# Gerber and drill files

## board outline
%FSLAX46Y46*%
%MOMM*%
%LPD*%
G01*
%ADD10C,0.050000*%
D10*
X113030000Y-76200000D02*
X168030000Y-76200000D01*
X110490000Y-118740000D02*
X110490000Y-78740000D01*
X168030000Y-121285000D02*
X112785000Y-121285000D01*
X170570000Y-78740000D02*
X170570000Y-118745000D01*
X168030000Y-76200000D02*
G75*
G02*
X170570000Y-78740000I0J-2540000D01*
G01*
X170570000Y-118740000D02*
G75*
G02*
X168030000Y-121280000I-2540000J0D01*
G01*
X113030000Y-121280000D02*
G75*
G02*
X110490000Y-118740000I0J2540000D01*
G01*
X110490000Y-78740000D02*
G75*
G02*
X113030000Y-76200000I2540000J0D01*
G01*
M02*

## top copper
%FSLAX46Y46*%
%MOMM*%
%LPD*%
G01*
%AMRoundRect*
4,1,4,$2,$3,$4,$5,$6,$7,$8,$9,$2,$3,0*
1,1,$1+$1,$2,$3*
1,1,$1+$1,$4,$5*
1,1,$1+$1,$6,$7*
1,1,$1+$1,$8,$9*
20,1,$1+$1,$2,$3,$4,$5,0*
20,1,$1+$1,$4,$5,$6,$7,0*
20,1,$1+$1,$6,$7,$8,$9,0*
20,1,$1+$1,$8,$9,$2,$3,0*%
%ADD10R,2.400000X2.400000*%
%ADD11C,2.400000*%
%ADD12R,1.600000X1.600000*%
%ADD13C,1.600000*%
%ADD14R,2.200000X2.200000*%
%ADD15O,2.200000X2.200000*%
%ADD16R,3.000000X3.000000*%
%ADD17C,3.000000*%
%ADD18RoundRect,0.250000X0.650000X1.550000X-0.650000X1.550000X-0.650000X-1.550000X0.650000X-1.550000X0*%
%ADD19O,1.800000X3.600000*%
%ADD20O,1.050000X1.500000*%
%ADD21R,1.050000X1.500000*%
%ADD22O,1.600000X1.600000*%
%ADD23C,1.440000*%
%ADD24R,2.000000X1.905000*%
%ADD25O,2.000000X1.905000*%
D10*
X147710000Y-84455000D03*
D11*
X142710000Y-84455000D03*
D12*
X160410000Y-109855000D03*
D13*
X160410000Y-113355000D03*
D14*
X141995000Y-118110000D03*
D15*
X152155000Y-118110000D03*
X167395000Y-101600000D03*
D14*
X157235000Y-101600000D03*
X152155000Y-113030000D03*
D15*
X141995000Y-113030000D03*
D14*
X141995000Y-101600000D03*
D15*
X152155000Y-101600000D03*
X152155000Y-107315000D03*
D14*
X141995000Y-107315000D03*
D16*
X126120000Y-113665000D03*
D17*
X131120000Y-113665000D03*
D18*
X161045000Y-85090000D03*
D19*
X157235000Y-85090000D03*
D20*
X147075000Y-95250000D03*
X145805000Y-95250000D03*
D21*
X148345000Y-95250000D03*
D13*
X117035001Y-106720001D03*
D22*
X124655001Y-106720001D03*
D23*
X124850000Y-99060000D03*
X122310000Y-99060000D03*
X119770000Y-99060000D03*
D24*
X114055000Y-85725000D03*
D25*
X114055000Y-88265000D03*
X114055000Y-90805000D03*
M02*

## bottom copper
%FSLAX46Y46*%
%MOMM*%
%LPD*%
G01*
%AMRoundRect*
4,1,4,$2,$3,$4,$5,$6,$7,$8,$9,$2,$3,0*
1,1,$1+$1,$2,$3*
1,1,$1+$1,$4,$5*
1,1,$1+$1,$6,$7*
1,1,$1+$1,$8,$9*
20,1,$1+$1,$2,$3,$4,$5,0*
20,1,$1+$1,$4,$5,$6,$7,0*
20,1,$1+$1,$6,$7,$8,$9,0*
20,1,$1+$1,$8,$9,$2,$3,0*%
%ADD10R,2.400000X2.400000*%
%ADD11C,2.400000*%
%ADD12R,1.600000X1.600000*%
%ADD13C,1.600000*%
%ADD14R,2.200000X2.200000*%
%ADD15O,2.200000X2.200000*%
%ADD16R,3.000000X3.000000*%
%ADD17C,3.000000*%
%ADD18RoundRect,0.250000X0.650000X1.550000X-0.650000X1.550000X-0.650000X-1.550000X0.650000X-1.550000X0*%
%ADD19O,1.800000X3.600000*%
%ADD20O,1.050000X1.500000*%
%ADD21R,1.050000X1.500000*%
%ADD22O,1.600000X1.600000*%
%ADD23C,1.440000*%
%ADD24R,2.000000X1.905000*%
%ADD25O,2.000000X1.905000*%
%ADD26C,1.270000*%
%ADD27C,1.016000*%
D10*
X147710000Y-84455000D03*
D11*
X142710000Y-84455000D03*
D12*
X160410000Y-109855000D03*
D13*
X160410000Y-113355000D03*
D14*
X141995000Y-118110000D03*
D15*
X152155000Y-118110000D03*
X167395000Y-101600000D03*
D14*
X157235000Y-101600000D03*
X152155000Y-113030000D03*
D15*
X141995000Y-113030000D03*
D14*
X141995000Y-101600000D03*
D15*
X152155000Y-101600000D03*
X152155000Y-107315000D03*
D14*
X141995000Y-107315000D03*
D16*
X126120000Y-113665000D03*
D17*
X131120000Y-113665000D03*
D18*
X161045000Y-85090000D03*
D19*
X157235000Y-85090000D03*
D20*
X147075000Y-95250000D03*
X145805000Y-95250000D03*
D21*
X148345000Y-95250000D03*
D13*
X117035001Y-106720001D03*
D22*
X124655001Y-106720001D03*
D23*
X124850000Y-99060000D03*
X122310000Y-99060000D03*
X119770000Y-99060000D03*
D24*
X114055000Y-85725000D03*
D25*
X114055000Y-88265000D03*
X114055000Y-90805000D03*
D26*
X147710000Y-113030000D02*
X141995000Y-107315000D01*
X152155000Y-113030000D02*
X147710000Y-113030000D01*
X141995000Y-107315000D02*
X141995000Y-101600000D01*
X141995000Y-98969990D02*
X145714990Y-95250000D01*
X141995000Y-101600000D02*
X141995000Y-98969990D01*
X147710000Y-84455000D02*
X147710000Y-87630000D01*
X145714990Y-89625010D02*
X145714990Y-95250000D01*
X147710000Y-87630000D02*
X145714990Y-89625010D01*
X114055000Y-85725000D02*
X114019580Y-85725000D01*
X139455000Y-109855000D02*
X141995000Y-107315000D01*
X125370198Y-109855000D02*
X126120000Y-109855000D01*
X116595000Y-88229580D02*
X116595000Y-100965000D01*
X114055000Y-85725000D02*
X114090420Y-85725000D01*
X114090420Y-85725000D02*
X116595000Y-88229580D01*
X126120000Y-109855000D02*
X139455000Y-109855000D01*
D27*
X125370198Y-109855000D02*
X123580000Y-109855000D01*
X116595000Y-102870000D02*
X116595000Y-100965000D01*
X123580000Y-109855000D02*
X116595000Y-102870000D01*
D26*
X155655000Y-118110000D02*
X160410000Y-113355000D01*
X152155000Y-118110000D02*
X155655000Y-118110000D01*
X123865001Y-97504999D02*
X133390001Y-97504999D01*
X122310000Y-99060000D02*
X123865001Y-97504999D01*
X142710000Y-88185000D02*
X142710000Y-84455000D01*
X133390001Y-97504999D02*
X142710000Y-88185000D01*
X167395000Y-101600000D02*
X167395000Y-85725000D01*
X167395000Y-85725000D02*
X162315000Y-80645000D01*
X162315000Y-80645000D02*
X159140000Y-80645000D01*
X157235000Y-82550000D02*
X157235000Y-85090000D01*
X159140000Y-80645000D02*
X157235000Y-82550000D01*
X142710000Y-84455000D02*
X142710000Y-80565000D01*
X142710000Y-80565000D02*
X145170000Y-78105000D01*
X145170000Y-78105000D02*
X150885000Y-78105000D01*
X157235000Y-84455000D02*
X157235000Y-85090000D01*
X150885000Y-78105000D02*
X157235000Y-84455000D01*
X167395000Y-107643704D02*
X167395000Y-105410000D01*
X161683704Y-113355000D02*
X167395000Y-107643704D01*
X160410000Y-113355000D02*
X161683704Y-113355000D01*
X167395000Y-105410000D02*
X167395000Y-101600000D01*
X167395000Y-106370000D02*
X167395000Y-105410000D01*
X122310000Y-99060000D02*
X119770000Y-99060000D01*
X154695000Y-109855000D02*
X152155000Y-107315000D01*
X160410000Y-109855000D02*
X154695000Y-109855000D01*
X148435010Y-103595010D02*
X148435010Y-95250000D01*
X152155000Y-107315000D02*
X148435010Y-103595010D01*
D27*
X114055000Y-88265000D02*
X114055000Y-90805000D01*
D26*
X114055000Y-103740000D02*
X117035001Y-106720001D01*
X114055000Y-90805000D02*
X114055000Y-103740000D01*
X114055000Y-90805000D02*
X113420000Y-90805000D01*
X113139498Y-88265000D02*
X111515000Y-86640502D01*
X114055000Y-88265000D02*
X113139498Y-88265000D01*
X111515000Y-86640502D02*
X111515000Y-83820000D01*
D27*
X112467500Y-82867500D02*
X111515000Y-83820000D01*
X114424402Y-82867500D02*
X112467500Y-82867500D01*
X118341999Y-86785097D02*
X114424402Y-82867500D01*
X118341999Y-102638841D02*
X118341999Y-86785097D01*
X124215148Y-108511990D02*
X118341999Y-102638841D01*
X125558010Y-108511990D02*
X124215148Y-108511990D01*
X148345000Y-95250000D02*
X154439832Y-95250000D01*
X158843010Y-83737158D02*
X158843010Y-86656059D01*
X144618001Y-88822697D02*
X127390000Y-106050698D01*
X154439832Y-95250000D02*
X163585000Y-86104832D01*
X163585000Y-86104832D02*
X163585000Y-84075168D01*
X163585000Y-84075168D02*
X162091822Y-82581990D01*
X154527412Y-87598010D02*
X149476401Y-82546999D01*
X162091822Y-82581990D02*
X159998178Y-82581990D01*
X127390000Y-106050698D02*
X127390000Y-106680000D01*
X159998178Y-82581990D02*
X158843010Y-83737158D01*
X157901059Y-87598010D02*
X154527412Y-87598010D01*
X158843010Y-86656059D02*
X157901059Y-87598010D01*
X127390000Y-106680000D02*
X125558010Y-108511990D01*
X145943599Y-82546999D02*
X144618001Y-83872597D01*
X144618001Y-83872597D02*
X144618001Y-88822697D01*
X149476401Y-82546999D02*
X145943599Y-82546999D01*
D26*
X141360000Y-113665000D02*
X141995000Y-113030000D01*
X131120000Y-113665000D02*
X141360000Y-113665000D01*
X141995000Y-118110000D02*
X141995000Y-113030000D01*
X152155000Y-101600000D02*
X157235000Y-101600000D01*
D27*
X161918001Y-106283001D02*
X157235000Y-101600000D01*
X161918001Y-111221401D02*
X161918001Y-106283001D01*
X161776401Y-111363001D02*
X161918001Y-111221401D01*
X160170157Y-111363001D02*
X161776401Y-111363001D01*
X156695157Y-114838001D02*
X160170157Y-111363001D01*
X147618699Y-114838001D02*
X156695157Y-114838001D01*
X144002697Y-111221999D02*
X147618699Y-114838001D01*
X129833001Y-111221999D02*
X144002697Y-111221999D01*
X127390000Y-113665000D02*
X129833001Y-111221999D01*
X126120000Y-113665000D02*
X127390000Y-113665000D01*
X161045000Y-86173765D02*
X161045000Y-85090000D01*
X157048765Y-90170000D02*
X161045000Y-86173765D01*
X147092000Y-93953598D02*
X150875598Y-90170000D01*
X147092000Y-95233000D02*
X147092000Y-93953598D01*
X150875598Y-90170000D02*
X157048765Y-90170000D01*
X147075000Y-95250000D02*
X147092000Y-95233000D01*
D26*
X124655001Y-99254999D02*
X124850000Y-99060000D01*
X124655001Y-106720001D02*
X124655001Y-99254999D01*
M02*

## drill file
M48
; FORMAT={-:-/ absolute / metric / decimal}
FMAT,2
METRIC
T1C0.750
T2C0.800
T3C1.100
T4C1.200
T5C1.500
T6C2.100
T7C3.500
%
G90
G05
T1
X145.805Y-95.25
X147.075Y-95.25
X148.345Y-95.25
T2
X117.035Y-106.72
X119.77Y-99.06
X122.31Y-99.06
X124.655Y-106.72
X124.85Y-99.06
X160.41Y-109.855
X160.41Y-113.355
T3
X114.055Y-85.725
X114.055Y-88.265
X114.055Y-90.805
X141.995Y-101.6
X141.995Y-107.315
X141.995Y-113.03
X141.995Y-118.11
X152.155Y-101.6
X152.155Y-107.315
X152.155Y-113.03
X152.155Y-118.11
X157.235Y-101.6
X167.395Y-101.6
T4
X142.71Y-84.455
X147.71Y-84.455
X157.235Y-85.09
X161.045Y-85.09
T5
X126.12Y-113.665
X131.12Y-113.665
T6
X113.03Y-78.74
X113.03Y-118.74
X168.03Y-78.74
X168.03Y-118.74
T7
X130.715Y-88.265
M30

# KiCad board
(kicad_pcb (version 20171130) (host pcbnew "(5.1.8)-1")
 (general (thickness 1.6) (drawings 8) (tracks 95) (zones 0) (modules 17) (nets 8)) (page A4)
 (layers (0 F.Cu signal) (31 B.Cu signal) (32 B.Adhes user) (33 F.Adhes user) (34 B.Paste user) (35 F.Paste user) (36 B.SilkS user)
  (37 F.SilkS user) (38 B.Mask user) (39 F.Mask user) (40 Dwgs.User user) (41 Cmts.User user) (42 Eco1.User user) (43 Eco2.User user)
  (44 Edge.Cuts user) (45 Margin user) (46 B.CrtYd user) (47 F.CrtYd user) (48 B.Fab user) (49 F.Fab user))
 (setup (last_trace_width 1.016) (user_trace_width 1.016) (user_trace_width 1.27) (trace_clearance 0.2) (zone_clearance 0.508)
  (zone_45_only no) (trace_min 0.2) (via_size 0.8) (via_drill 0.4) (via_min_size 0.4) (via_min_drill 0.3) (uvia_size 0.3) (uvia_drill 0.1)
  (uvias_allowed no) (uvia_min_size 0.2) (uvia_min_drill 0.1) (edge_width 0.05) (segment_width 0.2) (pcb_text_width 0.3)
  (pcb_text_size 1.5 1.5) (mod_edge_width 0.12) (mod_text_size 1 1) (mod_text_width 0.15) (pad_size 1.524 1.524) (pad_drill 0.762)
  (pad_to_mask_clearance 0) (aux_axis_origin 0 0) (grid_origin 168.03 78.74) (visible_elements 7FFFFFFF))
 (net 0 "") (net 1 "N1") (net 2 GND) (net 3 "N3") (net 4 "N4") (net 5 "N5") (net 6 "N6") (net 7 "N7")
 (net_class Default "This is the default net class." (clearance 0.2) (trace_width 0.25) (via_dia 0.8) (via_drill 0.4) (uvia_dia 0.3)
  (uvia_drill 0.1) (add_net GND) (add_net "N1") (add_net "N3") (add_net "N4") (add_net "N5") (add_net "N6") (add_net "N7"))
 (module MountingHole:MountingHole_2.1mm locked (layer F.Cu) (at 168.03 118.74)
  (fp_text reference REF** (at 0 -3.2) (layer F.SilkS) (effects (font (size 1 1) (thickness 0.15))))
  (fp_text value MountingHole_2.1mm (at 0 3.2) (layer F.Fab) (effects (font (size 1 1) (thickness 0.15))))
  (pad "" np_thru_hole circle (at 0 0) (size 2.1 2.1) (drill 2.1) (layers *.Cu *.Mask)))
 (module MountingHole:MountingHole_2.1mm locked (layer F.Cu) (at 113.03 118.74)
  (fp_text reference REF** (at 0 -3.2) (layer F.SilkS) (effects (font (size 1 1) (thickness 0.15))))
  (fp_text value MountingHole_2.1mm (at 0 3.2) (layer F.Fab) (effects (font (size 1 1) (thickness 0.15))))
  (pad "" np_thru_hole circle (at 0 0) (size 2.1 2.1) (drill 2.1) (layers *.Cu *.Mask)))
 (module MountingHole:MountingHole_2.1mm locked (layer F.Cu) (at 168.03 78.74)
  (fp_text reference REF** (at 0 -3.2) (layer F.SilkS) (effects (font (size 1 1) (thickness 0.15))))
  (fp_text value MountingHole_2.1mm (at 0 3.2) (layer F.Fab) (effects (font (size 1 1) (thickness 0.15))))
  (pad "" np_thru_hole circle (at 0 0) (size 2.1 2.1) (drill 2.1) (layers *.Cu *.Mask)))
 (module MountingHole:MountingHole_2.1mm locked (layer F.Cu) (at 113.03 78.74)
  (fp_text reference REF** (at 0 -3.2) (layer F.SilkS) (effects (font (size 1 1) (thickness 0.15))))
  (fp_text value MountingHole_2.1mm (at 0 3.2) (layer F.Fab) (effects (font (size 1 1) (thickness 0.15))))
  (pad "" np_thru_hole circle (at 0 0) (size 2.1 2.1) (drill 2.1) (layers *.Cu *.Mask)))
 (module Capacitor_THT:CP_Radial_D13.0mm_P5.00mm (layer F.Cu) (at 147.71 84.455 180)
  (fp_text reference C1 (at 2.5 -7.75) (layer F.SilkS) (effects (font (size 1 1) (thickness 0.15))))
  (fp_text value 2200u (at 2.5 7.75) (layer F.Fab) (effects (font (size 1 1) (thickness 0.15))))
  (pad 1 thru_hole rect (at 0 0 180) (size 2.4 2.4) (drill 1.2) (layers *.Cu *.Mask) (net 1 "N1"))
  (pad 2 thru_hole circle (at 5 0 180) (size 2.4 2.4) (drill 1.2) (layers *.Cu *.Mask) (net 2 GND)))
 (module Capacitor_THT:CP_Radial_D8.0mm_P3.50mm (layer F.Cu) (at 160.41 109.855 270)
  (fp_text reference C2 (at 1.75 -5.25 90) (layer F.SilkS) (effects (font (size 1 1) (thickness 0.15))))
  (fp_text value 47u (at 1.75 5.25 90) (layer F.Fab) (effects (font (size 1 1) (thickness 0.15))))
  (pad 1 thru_hole rect (at 0 0 270) (size 1.6 1.6) (drill 0.8) (layers *.Cu *.Mask) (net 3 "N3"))
  (pad 2 thru_hole circle (at 3.5 0 270) (size 1.6 1.6) (drill 0.8) (layers *.Cu *.Mask) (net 2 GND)))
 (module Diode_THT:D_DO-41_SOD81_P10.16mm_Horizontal (layer F.Cu) (at 141.995 118.11)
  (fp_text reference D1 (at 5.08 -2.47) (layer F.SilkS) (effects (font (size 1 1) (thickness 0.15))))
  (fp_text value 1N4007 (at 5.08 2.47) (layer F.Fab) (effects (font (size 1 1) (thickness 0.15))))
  (pad 1 thru_hole rect (at 0 0) (size 2.2 2.2) (drill 1.1) (layers *.Cu *.Mask) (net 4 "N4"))
  (pad 2 thru_hole oval (at 10.16 0) (size 2.2 2.2) (drill 1.1) (layers *.Cu *.Mask) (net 2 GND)))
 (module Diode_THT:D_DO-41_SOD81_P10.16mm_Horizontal (layer F.Cu) (at 157.235 101.6)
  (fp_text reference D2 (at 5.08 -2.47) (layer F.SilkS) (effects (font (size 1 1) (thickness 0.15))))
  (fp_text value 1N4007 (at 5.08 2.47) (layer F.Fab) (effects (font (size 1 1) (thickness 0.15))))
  (pad 2 thru_hole oval (at 10.16 0) (size 2.2 2.2) (drill 1.1) (layers *.Cu *.Mask) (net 2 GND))
  (pad 1 thru_hole rect (at 0 0) (size 2.2 2.2) (drill 1.1) (layers *.Cu *.Mask) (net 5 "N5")))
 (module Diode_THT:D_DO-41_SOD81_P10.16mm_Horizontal (layer F.Cu) (at 152.155 113.03 180)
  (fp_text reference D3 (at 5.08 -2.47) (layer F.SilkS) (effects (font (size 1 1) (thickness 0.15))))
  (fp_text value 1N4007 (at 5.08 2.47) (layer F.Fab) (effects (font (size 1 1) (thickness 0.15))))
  (pad 1 thru_hole rect (at 0 0 180) (size 2.2 2.2) (drill 1.1) (layers *.Cu *.Mask) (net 1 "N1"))
  (pad 2 thru_hole oval (at 10.16 0 180) (size 2.2 2.2) (drill 1.1) (layers *.Cu *.Mask) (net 4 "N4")))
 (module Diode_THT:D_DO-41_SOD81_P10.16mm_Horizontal (layer F.Cu) (at 141.995 101.6)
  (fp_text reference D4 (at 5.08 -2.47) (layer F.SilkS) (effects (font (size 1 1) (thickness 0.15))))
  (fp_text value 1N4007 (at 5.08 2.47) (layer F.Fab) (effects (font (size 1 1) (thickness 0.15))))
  (pad 1 thru_hole rect (at 0 0) (size 2.2 2.2) (drill 1.1) (layers *.Cu *.Mask) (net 1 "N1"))
  (pad 2 thru_hole oval (at 10.16 0) (size 2.2 2.2) (drill 1.1) (layers *.Cu *.Mask) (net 5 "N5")))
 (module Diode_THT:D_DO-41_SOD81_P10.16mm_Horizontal (layer F.Cu) (at 141.995 107.315)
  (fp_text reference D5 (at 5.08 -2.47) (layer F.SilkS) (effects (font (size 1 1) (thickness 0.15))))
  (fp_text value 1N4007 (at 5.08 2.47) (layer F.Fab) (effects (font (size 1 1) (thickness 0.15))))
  (pad 2 thru_hole oval (at 10.16 0) (size 2.2 2.2) (drill 1.1) (layers *.Cu *.Mask) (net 3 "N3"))
  (pad 1 thru_hole rect (at 0 0) (size 2.2 2.2) (drill 1.1) (layers *.Cu *.Mask) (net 1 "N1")))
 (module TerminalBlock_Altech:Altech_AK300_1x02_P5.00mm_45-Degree (layer F.Cu) (at 126.12 113.665)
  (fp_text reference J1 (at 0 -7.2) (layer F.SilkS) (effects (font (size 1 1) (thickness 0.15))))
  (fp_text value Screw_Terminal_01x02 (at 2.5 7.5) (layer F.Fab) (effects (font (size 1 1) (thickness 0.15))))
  (pad 1 thru_hole rect (at 0 0) (size 3 3) (drill 1.5) (layers *.Cu *.Mask) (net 5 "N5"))
  (pad 2 thru_hole circle (at 5 0) (size 3 3) (drill 1.5) (layers *.Cu *.Mask) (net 4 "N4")))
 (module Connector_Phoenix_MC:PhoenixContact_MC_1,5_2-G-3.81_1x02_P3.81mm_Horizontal (layer F.Cu) (at 161.045 85.09 180)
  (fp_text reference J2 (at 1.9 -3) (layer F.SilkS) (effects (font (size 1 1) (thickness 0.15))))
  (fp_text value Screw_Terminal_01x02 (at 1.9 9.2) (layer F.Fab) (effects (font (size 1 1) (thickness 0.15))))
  (pad 1 thru_hole roundrect (at 0 0 180) (size 1.8 3.6) (drill 1.2) (layers *.Cu *.Mask) (roundrect_rratio 0.1388888888888889) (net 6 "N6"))
  (pad 2 thru_hole oval (at 3.81 0 180) (size 1.8 3.6) (drill 1.2) (layers *.Cu *.Mask) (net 2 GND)))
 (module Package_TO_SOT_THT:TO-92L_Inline (layer F.Cu) (at 148.345 95.25 180)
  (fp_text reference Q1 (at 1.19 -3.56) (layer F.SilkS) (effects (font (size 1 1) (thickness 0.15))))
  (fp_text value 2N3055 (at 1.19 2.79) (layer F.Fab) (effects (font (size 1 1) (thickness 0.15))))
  (pad 2 thru_hole oval (at 1.27 0 180) (size 1.05 1.5) (drill 0.75) (layers *.Cu *.Mask) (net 6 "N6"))
  (pad 3 thru_hole oval (at 2.54 0 180) (size 1.05 1.5) (drill 0.75) (layers *.Cu *.Mask) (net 1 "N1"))
  (pad 1 thru_hole rect (at 0 0 180) (size 1.05 1.5) (drill 0.75) (layers *.Cu *.Mask) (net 3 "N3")))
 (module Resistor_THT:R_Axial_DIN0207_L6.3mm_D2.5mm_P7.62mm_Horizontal (layer F.Cu) (at 117.035001 106.720001)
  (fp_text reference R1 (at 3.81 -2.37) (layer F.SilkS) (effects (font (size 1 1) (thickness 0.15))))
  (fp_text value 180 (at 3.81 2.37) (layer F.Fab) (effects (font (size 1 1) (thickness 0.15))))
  (pad 1 thru_hole circle (at 0 0) (size 1.6 1.6) (drill 0.8) (layers *.Cu *.Mask) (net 3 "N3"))
  (pad 2 thru_hole oval (at 7.62 0) (size 1.6 1.6) (drill 0.8) (layers *.Cu *.Mask) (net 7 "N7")))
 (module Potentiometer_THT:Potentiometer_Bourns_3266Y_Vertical (layer F.Cu) (at 124.85 99.06)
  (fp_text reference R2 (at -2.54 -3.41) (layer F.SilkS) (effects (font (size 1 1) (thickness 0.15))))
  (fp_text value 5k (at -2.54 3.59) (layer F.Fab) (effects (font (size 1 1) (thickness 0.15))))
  (pad 1 thru_hole circle (at 0 0) (size 1.44 1.44) (drill 0.8) (layers *.Cu *.Mask) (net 7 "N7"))
  (pad 2 thru_hole circle (at -2.54 0) (size 1.44 1.44) (drill 0.8) (layers *.Cu *.Mask) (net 2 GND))
  (pad 3 thru_hole circle (at -5.08 0) (size 1.44 1.44) (drill 0.8) (layers *.Cu *.Mask) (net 2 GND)))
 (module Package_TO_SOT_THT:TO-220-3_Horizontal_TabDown (layer F.Cu) (at 114.055 85.725 270)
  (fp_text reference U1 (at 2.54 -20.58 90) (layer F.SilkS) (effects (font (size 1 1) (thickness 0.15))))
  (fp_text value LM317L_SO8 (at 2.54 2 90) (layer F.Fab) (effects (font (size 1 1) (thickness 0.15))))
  (pad "" np_thru_hole oval (at 2.54 -16.66 270) (size 3.5 3.5) (drill 3.5) (layers *.Cu *.Mask))
  (pad 1 thru_hole rect (at 0 0 270) (size 1.905 2) (drill 1.1) (layers *.Cu *.Mask) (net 1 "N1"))
  (pad 2 thru_hole oval (at 2.54 0 270) (size 1.905 2) (drill 1.1) (layers *.Cu *.Mask) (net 3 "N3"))
  (pad 3 thru_hole oval (at 5.08 0 270) (size 1.905 2) (drill 1.1) (layers *.Cu *.Mask) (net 3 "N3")))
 (gr_line (start 113.03 76.2) (end 168.03 76.2) (layer Edge.Cuts) (width 0.05))
 (gr_line (start 110.49 118.74) (end 110.49 78.74) (layer Edge.Cuts) (width 0.05))
 (gr_line (start 168.03 121.285) (end 112.785 121.285) (layer Edge.Cuts) (width 0.05))
 (gr_line (start 170.57 78.74) (end 170.57 118.745) (layer Edge.Cuts) (width 0.05))
 (gr_arc (start 168.03 78.74) (end 170.57 78.74) (angle -90) (layer Edge.Cuts) (width 0.05))
 (gr_arc (start 168.03 118.74) (end 168.03 121.28) (angle -90) (layer Edge.Cuts) (width 0.05))
 (gr_arc (start 113.03 118.74) (end 110.49 118.74) (angle -90) (layer Edge.Cuts) (width 0.05))
 (gr_arc (start 113.03 78.74) (end 113.03 76.2) (angle -90) (layer Edge.Cuts) (width 0.05))
 (segment (start 147.71 113.03) (end 141.995 107.315) (width 1.27) (layer B.Cu) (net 1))
 (segment (start 152.155 113.03) (end 147.71 113.03) (width 1.27) (layer B.Cu) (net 1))
 (segment (start 141.995 107.315) (end 141.995 101.6) (width 1.27) (layer B.Cu) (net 1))
 (segment (start 141.995 98.96999) (end 145.71499 95.25) (width 1.27) (layer B.Cu) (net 1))
 (segment (start 141.995 101.6) (end 141.995 98.96999) (width 1.27) (layer B.Cu) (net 1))
 (segment (start 147.71 84.455) (end 147.71 87.63) (width 1.27) (layer B.Cu) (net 1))
 (segment (start 145.71499 89.62501) (end 145.71499 95.25) (width 1.27) (layer B.Cu) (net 1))
 (segment (start 147.71 87.63) (end 145.71499 89.62501) (width 1.27) (layer B.Cu) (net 1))
 (segment (start 114.055 85.725) (end 114.01958 85.725) (width 1.27) (layer B.Cu) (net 1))
 (segment (start 139.455 109.855) (end 141.995 107.315) (width 1.27) (layer B.Cu) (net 1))
 (segment (start 125.370198 109.855) (end 126.12 109.855) (width 1.27) (layer B.Cu) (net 1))
 (segment (start 116.595 88.22958) (end 116.595 100.965) (width 1.27) (layer B.Cu) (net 1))
 (segment (start 114.055 85.725) (end 114.09042 85.725) (width 1.27) (layer B.Cu) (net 1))
 (segment (start 114.09042 85.725) (end 116.595 88.22958) (width 1.27) (layer B.Cu) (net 1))
 (segment (start 126.12 109.855) (end 139.455 109.855) (width 1.27) (layer B.Cu) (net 1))
 (segment (start 125.370198 109.855) (end 123.58 109.855) (width 1.016) (layer B.Cu) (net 1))
 (segment (start 116.595 102.87) (end 116.595 100.965) (width 1.016) (layer B.Cu) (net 1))
 (segment (start 123.58 109.855) (end 116.595 102.87) (width 1.016) (layer B.Cu) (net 1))
 (segment (start 155.655 118.11) (end 160.41 113.355) (width 1.27) (layer B.Cu) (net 2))
 (segment (start 152.155 118.11) (end 155.655 118.11) (width 1.27) (layer B.Cu) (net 2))
 (segment (start 123.865001 97.504999) (end 133.390001 97.504999) (width 1.27) (layer B.Cu) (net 2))
 (segment (start 122.31 99.06) (end 123.865001 97.504999) (width 1.27) (layer B.Cu) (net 2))
 (segment (start 142.71 88.185) (end 142.71 84.455) (width 1.27) (layer B.Cu) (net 2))
 (segment (start 133.390001 97.504999) (end 142.71 88.185) (width 1.27) (layer B.Cu) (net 2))
 (segment (start 167.395 101.6) (end 167.395 85.725) (width 1.27) (layer B.Cu) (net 2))
 (segment (start 167.395 85.725) (end 162.315 80.645) (width 1.27) (layer B.Cu) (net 2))
 (segment (start 162.315 80.645) (end 159.14 80.645) (width 1.27) (layer B.Cu) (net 2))
 (segment (start 157.235 82.55) (end 157.235 85.09) (width 1.27) (layer B.Cu) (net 2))
 (segment (start 159.14 80.645) (end 157.235 82.55) (width 1.27) (layer B.Cu) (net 2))
 (segment (start 142.71 84.455) (end 142.71 80.565) (width 1.27) (layer B.Cu) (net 2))
 (segment (start 142.71 80.565) (end 145.17 78.105) (width 1.27) (layer B.Cu) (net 2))
 (segment (start 145.17 78.105) (end 150.885 78.105) (width 1.27) (layer B.Cu) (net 2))
 (segment (start 157.235 84.455) (end 157.235 85.09) (width 1.27) (layer B.Cu) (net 2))
 (segment (start 150.885 78.105) (end 157.235 84.455) (width 1.27) (layer B.Cu) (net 2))
 (segment (start 167.395 107.643704) (end 167.395 105.41) (width 1.27) (layer B.Cu) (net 2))
 (segment (start 161.683704 113.355) (end 167.395 107.643704) (width 1.27) (layer B.Cu) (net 2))
 (segment (start 160.41 113.355) (end 161.683704 113.355) (width 1.27) (layer B.Cu) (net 2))
 (segment (start 167.395 105.41) (end 167.395 101.6) (width 1.27) (layer B.Cu) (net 2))
 (segment (start 167.395 106.37) (end 167.395 105.41) (width 1.27) (layer B.Cu) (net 2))
 (segment (start 122.31 99.06) (end 119.77 99.06) (width 1.27) (layer B.Cu) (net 2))
 (segment (start 154.695 109.855) (end 152.155 107.315) (width 1.27) (layer B.Cu) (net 3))
 (segment (start 160.41 109.855) (end 154.695 109.855) (width 1.27) (layer B.Cu) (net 3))
 (segment (start 148.43501 103.59501) (end 148.43501 95.25) (width 1.27) (layer B.Cu) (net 3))
 (segment (start 152.155 107.315) (end 148.43501 103.59501) (width 1.27) (layer B.Cu) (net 3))
 (segment (start 114.055 88.265) (end 114.055 90.805) (width 1.016) (layer B.Cu) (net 3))
 (segment (start 114.055 103.74) (end 117.035001 106.720001) (width 1.27) (layer B.Cu) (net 3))
 (segment (start 114.055 90.805) (end 114.055 103.74) (width 1.27) (layer B.Cu) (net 3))
 (segment (start 114.055 90.805) (end 113.42 90.805) (width 1.27) (layer B.Cu) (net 3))
 (segment (start 113.139498 88.265) (end 111.515 86.640502) (width 1.27) (layer B.Cu) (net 3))
 (segment (start 114.055 88.265) (end 113.139498 88.265) (width 1.27) (layer B.Cu) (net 3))
 (segment (start 111.515 86.640502) (end 111.515 83.82) (width 1.27) (layer B.Cu) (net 3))
 (segment (start 112.4675 82.8675) (end 111.515 83.82) (width 1.016) (layer B.Cu) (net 3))
 (segment (start 114.424402 82.8675) (end 112.4675 82.8675) (width 1.016) (layer B.Cu) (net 3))
 (segment (start 118.341999 86.785097) (end 114.424402 82.8675) (width 1.016) (layer B.Cu) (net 3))
 (segment (start 118.341999 102.638841) (end 118.341999 86.785097) (width 1.016) (layer B.Cu) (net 3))
 (segment (start 124.215148 108.51199) (end 118.341999 102.638841) (width 1.016) (layer B.Cu) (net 3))
 (segment (start 125.55801 108.51199) (end 124.215148 108.51199) (width 1.016) (layer B.Cu) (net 3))
 (segment (start 148.345 95.25) (end 154.439832 95.25) (width 1.016) (layer B.Cu) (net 3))
 (segment (start 158.84301 83.737158) (end 158.84301 86.656059) (width 1.016) (layer B.Cu) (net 3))
 (segment (start 144.618001 88.822697) (end 127.39 106.050698) (width 1.016) (layer B.Cu) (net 3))
 (segment (start 154.439832 95.25) (end 163.585 86.104832) (width 1.016) (layer B.Cu) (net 3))
 (segment (start 163.585 86.104832) (end 163.585 84.075168) (width 1.016) (layer B.Cu) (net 3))
 (segment (start 163.585 84.075168) (end 162.091822 82.58199) (width 1.016) (layer B.Cu) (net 3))
 (segment (start 154.527412 87.59801) (end 149.476401 82.546999) (width 1.016) (layer B.Cu) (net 3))
 (segment (start 162.091822 82.58199) (end 159.998178 82.58199) (width 1.016) (layer B.Cu) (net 3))
 (segment (start 127.39 106.050698) (end 127.39 106.68) (width 1.016) (layer B.Cu) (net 3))
 (segment (start 159.998178 82.58199) (end 158.84301 83.737158) (width 1.016) (layer B.Cu) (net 3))
 (segment (start 157.901059 87.59801) (end 154.527412 87.59801) (width 1.016) (layer B.Cu) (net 3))
 (segment (start 158.84301 86.656059) (end 157.901059 87.59801) (width 1.016) (layer B.Cu) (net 3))
 (segment (start 127.39 106.68) (end 125.55801 108.51199) (width 1.016) (layer B.Cu) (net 3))
 (segment (start 145.943599 82.546999) (end 144.618001 83.872597) (width 1.016) (layer B.Cu) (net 3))
 (segment (start 144.618001 83.872597) (end 144.618001 88.822697) (width 1.016) (layer B.Cu) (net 3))
 (segment (start 149.476401 82.546999) (end 145.943599 82.546999) (width 1.016) (layer B.Cu) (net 3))
 (segment (start 141.36 113.665) (end 141.995 113.03) (width 1.27) (layer B.Cu) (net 4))
 (segment (start 131.12 113.665) (end 141.36 113.665) (width 1.27) (layer B.Cu) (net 4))
 (segment (start 141.995 118.11) (end 141.995 113.03) (width 1.27) (layer B.Cu) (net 4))
 (segment (start 152.155 101.6) (end 157.235 101.6) (width 1.27) (layer B.Cu) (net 5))
 (segment (start 161.918001 106.283001) (end 157.235 101.6) (width 1.016) (layer B.Cu) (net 5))
 (segment (start 161.918001 111.221401) (end 161.918001 106.283001) (width 1.016) (layer B.Cu) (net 5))
 (segment (start 161.776401 111.363001) (end 161.918001 111.221401) (width 1.016) (layer B.Cu) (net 5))
 (segment (start 160.170157 111.363001) (end 161.776401 111.363001) (width 1.016) (layer B.Cu) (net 5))
 (segment (start 156.695157 114.838001) (end 160.170157 111.363001) (width 1.016) (layer B.Cu) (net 5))
 (segment (start 147.618699 114.838001) (end 156.695157 114.838001) (width 1.016) (layer B.Cu) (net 5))
 (segment (start 144.002697 111.221999) (end 147.618699 114.838001) (width 1.016) (layer B.Cu) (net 5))
 (segment (start 129.833001 111.221999) (end 144.002697 111.221999) (width 1.016) (layer B.Cu) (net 5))
 (segment (start 127.39 113.665) (end 129.833001 111.221999) (width 1.016) (layer B.Cu) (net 5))
 (segment (start 126.12 113.665) (end 127.39 113.665) (width 1.016) (layer B.Cu) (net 5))
 (segment (start 161.045 86.173765) (end 161.045 85.09) (width 1.016) (layer B.Cu) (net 6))
 (segment (start 157.048765 90.17) (end 161.045 86.173765) (width 1.016) (layer B.Cu) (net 6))
 (segment (start 147.092 93.953598) (end 150.875598 90.17) (width 1.016) (layer B.Cu) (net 6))
 (segment (start 147.092 95.233) (end 147.092 93.953598) (width 1.016) (layer B.Cu) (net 6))
 (segment (start 150.875598 90.17) (end 157.048765 90.17) (width 1.016) (layer B.Cu) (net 6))
 (segment (start 147.075 95.25) (end 147.092 95.233) (width 1.016) (layer B.Cu) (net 6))
 (segment (start 124.655001 99.254999) (end 124.85 99.06) (width 1.27) (layer B.Cu) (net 7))
 (segment (start 124.655001 106.720001) (end 124.655001 99.254999) (width 1.27) (layer B.Cu) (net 7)))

